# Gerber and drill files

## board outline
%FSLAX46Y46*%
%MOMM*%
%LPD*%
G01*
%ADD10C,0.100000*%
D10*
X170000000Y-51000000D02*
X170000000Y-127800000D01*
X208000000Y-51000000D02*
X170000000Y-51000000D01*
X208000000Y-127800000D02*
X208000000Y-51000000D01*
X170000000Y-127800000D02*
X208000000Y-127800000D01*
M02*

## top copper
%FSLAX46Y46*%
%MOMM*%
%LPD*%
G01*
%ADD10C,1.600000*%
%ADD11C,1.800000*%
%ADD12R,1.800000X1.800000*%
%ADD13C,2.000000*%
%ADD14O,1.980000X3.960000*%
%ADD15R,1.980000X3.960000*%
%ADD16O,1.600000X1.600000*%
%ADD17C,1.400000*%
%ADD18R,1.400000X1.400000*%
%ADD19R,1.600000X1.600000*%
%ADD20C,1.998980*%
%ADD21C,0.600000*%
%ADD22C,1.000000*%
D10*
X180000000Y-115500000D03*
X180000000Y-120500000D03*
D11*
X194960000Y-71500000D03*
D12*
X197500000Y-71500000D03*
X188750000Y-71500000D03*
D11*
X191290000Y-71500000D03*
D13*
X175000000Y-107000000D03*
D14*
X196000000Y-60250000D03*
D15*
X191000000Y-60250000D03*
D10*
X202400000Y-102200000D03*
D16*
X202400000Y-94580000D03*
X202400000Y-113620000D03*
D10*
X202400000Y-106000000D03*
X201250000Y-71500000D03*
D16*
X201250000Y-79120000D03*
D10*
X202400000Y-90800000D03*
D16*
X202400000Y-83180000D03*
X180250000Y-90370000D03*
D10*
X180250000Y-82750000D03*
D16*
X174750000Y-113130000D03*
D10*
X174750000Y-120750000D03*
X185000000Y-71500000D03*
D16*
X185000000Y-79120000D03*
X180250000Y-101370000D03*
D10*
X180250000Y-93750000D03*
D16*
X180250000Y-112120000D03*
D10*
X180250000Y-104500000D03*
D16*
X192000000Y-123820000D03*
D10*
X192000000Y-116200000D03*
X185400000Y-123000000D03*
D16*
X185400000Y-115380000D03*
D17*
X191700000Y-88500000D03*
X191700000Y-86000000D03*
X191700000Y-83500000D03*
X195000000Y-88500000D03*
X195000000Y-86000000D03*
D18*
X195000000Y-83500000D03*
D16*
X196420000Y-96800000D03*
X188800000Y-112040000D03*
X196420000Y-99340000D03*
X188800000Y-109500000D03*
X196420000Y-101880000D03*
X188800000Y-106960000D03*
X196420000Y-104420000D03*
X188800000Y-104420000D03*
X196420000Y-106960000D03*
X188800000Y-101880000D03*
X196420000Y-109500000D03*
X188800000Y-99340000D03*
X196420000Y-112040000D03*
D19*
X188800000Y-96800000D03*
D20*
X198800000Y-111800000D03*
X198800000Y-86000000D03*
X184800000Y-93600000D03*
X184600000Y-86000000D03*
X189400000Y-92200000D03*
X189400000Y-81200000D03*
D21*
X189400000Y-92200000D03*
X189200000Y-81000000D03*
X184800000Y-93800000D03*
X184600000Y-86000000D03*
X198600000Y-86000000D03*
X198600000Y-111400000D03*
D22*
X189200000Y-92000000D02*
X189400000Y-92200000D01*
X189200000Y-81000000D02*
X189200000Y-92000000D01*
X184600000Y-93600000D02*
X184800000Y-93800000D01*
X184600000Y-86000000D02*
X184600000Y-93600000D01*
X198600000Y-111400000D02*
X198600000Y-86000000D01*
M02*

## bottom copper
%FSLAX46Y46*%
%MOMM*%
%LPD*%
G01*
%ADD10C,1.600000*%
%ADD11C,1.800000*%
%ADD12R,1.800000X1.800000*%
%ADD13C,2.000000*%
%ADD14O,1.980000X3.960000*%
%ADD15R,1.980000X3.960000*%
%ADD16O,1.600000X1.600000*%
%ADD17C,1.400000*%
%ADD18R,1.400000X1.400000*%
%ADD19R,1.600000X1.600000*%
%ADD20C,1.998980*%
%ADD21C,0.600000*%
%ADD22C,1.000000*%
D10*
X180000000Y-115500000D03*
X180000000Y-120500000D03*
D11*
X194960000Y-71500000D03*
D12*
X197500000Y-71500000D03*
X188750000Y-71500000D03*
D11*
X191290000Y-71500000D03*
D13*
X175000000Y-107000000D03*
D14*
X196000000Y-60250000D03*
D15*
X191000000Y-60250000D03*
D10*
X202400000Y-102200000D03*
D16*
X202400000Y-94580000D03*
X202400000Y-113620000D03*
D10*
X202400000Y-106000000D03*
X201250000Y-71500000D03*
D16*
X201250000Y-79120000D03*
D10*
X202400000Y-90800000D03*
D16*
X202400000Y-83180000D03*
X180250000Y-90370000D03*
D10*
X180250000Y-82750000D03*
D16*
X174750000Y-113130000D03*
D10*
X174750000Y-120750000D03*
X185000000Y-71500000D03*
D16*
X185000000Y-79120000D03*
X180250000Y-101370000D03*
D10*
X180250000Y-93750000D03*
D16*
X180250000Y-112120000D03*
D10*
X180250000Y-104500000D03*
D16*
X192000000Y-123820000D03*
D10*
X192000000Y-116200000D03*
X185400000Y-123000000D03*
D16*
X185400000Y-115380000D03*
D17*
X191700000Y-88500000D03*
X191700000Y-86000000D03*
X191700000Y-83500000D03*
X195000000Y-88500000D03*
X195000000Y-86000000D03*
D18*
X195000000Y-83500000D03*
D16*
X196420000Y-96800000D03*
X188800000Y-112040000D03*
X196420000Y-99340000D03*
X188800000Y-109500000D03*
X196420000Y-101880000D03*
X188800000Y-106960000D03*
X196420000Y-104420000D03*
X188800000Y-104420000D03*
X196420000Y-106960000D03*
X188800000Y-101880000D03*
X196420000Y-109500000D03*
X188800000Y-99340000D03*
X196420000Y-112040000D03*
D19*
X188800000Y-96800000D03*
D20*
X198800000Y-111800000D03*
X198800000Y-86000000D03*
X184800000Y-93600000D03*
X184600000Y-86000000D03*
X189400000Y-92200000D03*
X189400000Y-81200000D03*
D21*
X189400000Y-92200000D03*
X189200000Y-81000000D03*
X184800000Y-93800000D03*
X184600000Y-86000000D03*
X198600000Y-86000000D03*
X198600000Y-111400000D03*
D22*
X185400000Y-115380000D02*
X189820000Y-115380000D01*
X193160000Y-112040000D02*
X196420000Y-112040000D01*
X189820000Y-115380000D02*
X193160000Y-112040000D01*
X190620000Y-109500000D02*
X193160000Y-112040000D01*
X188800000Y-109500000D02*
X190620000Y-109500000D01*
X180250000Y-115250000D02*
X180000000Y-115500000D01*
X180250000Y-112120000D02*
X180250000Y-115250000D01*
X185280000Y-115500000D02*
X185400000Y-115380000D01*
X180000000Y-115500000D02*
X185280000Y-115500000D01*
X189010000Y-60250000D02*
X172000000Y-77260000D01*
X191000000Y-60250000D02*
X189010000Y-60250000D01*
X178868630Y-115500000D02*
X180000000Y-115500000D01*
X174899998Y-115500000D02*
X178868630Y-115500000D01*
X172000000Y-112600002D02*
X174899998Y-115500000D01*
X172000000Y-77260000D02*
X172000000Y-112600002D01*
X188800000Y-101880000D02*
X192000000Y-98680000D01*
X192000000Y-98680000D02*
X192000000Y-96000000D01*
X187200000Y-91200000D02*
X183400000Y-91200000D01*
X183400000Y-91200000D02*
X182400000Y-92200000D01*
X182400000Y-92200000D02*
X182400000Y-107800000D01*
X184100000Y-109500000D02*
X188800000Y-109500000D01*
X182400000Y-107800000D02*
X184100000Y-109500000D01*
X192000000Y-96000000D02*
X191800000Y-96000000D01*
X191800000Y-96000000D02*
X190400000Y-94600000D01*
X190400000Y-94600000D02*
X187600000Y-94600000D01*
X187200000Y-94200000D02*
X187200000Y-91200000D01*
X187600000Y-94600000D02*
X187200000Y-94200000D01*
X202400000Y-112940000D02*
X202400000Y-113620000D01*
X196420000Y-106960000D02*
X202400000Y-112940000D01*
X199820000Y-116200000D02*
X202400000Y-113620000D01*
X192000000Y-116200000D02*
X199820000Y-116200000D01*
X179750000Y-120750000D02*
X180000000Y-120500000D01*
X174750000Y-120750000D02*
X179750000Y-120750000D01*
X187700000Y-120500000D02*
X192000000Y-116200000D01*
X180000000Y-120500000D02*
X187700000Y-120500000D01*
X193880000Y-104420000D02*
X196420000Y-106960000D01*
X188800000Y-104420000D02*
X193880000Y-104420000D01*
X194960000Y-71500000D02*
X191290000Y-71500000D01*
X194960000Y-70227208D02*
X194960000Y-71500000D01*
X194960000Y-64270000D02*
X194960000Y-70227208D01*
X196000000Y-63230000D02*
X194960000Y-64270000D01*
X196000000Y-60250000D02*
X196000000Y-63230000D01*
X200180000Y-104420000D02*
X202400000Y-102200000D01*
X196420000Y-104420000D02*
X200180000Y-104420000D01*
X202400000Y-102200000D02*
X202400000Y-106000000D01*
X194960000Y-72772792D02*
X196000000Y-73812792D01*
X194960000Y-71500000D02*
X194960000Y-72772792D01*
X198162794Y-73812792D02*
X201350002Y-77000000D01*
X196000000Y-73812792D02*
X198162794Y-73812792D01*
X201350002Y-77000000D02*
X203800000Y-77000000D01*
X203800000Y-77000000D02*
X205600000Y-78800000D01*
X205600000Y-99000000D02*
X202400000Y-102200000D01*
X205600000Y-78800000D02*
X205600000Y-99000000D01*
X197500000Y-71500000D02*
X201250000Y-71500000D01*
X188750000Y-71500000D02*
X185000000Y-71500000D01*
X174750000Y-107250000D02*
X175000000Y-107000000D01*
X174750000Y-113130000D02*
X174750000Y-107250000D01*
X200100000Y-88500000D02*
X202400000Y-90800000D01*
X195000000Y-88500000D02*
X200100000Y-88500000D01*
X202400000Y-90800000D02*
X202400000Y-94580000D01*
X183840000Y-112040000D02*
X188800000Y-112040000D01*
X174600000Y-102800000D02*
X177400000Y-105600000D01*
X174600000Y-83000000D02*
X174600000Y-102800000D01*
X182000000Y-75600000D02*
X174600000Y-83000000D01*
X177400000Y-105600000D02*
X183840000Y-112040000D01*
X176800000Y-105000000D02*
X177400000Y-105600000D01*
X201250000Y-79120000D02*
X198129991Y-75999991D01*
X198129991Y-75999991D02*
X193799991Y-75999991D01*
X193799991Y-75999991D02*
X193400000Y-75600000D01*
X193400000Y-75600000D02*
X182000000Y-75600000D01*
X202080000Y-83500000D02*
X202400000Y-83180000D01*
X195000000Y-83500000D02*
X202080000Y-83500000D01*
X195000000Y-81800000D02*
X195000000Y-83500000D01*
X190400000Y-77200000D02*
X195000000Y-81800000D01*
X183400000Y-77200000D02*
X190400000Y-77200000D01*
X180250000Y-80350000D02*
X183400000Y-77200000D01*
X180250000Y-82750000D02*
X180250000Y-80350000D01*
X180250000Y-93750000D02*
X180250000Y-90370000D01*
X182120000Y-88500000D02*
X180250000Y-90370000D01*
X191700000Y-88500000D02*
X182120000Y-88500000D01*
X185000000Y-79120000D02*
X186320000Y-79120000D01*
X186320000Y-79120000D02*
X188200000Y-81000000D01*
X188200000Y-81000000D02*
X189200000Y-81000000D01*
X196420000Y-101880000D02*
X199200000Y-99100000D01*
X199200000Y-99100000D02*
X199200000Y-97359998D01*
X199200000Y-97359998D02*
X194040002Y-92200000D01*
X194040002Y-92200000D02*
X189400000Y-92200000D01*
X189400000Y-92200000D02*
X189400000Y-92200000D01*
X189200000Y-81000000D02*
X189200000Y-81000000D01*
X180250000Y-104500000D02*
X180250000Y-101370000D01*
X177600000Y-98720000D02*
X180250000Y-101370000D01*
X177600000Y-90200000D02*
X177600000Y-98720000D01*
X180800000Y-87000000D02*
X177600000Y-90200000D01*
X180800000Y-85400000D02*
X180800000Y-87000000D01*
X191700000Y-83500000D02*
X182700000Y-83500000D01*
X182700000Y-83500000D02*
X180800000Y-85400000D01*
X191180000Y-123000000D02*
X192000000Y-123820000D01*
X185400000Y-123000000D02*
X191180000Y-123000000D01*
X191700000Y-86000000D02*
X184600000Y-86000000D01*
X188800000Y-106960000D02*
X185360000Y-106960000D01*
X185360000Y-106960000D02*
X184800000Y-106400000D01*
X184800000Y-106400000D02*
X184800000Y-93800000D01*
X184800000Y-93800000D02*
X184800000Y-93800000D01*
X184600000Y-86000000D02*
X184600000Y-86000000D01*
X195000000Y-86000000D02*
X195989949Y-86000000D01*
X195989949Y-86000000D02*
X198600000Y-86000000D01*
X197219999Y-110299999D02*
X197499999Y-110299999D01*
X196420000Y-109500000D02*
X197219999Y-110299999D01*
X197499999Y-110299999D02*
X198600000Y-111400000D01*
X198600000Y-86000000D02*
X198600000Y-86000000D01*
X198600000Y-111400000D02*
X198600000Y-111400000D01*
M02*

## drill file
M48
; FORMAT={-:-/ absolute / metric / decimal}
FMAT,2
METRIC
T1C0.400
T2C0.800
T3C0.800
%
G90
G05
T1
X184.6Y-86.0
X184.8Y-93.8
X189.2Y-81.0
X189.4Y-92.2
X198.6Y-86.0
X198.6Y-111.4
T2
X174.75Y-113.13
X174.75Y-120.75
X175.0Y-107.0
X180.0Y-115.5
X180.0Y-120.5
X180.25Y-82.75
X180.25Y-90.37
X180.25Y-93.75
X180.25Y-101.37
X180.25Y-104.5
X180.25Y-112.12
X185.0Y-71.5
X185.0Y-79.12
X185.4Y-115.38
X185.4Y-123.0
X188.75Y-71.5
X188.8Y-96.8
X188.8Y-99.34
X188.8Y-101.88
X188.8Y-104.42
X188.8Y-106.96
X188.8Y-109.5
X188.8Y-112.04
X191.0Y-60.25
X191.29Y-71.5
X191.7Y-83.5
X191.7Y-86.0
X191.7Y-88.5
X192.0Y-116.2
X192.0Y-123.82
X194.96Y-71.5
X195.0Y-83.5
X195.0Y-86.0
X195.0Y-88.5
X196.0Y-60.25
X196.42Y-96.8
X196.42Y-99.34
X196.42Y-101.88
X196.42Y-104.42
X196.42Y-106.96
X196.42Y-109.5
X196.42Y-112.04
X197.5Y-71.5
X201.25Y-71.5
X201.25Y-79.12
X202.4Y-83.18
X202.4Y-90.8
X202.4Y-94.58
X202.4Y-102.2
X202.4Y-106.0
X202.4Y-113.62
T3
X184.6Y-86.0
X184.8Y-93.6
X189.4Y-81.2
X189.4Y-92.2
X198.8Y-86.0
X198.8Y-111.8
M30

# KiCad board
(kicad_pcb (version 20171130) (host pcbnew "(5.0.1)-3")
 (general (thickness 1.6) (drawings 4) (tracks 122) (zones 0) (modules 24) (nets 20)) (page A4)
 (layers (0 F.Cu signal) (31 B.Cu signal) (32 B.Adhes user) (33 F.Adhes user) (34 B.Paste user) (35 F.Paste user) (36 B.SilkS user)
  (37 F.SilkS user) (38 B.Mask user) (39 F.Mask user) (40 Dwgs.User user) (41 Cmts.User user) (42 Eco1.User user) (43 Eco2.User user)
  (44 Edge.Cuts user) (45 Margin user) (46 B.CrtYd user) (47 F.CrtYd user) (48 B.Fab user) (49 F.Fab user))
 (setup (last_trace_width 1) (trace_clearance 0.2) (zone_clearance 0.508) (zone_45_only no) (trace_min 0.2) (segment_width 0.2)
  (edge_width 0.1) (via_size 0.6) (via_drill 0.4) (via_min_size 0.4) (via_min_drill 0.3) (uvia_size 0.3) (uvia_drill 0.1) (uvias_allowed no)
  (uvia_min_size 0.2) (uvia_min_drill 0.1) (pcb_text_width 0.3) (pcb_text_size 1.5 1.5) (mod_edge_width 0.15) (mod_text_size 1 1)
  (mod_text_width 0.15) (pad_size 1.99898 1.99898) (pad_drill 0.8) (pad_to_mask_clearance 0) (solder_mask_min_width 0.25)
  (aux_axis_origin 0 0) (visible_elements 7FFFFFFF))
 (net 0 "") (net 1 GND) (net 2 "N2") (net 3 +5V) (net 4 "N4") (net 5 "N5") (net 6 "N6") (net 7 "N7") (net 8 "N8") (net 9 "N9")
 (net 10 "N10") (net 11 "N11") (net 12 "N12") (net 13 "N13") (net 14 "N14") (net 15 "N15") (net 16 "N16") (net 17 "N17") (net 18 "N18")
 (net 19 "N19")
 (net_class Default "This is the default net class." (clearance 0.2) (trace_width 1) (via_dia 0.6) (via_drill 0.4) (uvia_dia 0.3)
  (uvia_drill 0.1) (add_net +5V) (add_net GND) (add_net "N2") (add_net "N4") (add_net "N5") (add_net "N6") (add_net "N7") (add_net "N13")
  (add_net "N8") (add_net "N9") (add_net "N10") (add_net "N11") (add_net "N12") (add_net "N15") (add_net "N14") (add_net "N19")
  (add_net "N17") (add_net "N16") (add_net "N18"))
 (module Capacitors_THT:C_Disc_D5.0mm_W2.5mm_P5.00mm (layer F.Cu) (at 180 120.5 90)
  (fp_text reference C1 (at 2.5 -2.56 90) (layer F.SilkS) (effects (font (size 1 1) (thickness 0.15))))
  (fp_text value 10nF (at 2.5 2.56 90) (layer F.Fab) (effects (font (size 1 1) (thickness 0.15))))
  (pad 2 thru_hole circle (at 5 0 90) (size 1.6 1.6) (drill 0.8) (layers *.Cu *.Mask) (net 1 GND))
  (pad 1 thru_hole circle (at 0 0 90) (size 1.6 1.6) (drill 0.8) (layers *.Cu *.Mask) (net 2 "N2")))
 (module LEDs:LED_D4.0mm (layer F.Cu) (at 197.5 71.5 180)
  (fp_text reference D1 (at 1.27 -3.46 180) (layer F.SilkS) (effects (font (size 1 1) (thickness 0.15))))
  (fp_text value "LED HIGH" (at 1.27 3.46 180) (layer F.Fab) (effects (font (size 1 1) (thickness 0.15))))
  (pad 2 thru_hole circle (at 2.54 0 180) (size 1.8 1.8) (drill 0.8) (layers *.Cu *.Mask) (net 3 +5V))
  (pad 1 thru_hole rect (at 0 0 180) (size 1.8 1.8) (drill 0.8) (layers *.Cu *.Mask) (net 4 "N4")))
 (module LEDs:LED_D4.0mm (layer F.Cu) (at 188.75 71.5)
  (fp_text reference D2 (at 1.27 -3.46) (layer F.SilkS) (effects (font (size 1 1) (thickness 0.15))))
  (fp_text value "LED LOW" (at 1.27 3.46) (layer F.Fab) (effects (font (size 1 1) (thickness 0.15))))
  (pad 1 thru_hole rect (at 0 0) (size 1.8 1.8) (drill 0.8) (layers *.Cu *.Mask) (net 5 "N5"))
  (pad 2 thru_hole circle (at 2.54 0) (size 1.8 1.8) (drill 0.8) (layers *.Cu *.Mask) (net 3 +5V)))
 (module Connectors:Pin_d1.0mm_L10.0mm (layer F.Cu) (at 175 107)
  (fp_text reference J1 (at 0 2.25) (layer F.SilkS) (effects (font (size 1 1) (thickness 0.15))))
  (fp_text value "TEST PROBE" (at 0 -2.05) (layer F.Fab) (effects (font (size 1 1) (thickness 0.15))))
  (pad 1 thru_hole circle (at 0 0) (size 2 2) (drill 0.8) (layers *.Cu *.Mask) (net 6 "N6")))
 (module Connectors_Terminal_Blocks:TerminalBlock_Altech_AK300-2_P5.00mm (layer F.Cu) (at 191 60.25)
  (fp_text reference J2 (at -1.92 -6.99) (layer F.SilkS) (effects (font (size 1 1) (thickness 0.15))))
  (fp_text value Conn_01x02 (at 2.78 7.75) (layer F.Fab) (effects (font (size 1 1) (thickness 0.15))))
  (pad 2 thru_hole oval (at 5 0) (size 1.98 3.96) (drill 0.8) (layers *.Cu *.Mask) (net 3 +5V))
  (pad 1 thru_hole rect (at 0 0) (size 1.98 3.96) (drill 0.8) (layers *.Cu *.Mask) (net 1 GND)))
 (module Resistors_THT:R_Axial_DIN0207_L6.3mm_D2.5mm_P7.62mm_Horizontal (layer F.Cu) (at 202.4 102.2 90)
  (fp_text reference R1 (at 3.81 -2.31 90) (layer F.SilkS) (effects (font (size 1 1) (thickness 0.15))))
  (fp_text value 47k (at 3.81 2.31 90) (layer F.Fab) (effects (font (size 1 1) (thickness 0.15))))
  (pad 1 thru_hole circle (at 0 0 90) (size 1.6 1.6) (drill 0.8) (layers *.Cu *.Mask) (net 3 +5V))
  (pad 2 thru_hole oval (at 7.62 0 90) (size 1.6 1.6) (drill 0.8) (layers *.Cu *.Mask) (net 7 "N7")))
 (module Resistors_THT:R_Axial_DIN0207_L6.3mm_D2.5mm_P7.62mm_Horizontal (layer F.Cu) (at 202.4 106 270)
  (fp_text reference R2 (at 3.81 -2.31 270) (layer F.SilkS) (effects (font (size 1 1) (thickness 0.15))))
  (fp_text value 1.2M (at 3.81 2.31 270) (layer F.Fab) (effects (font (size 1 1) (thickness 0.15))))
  (pad 2 thru_hole oval (at 7.62 0 270) (size 1.6 1.6) (drill 0.8) (layers *.Cu *.Mask) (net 2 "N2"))
  (pad 1 thru_hole circle (at 0 0 270) (size 1.6 1.6) (drill 0.8) (layers *.Cu *.Mask) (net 3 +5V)))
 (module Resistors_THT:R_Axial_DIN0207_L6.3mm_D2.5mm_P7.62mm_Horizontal (layer F.Cu) (at 201.25 71.5 270)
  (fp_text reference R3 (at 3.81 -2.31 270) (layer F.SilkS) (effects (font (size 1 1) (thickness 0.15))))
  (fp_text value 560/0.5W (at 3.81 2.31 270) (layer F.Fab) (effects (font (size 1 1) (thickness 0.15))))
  (pad 1 thru_hole circle (at 0 0 270) (size 1.6 1.6) (drill 0.8) (layers *.Cu *.Mask) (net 4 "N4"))
  (pad 2 thru_hole oval (at 7.62 0 270) (size 1.6 1.6) (drill 0.8) (layers *.Cu *.Mask) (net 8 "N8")))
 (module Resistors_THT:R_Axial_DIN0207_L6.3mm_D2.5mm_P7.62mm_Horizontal (layer F.Cu) (at 202.4 90.8 90)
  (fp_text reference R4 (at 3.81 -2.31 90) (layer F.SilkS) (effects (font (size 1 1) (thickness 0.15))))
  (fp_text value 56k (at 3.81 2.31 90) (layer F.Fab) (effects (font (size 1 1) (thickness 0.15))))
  (pad 1 thru_hole circle (at 0 0 90) (size 1.6 1.6) (drill 0.8) (layers *.Cu *.Mask) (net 7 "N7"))
  (pad 2 thru_hole oval (at 7.62 0 90) (size 1.6 1.6) (drill 0.8) (layers *.Cu *.Mask) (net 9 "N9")))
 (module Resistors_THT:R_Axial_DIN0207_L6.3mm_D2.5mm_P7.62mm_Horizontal (layer F.Cu) (at 180.25 82.75 270)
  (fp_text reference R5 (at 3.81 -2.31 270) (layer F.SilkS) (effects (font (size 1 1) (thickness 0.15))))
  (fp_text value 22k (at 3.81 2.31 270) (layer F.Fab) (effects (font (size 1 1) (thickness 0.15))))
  (pad 2 thru_hole oval (at 7.62 0 270) (size 1.6 1.6) (drill 0.8) (layers *.Cu *.Mask) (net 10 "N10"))
  (pad 1 thru_hole circle (at 0 0 270) (size 1.6 1.6) (drill 0.8) (layers *.Cu *.Mask) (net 9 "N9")))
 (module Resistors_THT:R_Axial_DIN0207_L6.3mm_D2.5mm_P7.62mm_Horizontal (layer F.Cu) (at 174.75 120.75 90)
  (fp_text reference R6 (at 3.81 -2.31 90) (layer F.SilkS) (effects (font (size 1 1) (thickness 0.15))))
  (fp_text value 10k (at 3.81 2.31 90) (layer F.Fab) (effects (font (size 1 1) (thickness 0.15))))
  (pad 2 thru_hole oval (at 7.62 0 90) (size 1.6 1.6) (drill 0.8) (layers *.Cu *.Mask) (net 6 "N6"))
  (pad 1 thru_hole circle (at 0 0 90) (size 1.6 1.6) (drill 0.8) (layers *.Cu *.Mask) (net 2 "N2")))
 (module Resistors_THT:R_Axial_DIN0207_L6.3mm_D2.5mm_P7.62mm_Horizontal (layer F.Cu) (at 185 71.5 270)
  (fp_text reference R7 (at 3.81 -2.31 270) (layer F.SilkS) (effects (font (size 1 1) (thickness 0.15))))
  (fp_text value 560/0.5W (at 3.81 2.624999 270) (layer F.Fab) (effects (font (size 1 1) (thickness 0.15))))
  (pad 1 thru_hole circle (at 0 0 270) (size 1.6 1.6) (drill 0.8) (layers *.Cu *.Mask) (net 5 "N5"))
  (pad 2 thru_hole oval (at 7.62 0 270) (size 1.6 1.6) (drill 0.8) (layers *.Cu *.Mask) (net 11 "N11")))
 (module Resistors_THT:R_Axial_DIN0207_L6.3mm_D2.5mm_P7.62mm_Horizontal (layer F.Cu) (at 180.25 93.75 270)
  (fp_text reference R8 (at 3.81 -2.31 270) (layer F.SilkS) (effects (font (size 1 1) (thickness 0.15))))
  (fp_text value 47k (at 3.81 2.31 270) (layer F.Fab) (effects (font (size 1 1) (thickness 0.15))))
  (pad 2 thru_hole oval (at 7.62 0 270) (size 1.6 1.6) (drill 0.8) (layers *.Cu *.Mask) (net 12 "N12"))
  (pad 1 thru_hole circle (at 0 0 270) (size 1.6 1.6) (drill 0.8) (layers *.Cu *.Mask) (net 10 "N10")))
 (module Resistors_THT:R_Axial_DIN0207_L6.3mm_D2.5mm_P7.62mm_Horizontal (layer F.Cu) (at 180.25 104.5 270)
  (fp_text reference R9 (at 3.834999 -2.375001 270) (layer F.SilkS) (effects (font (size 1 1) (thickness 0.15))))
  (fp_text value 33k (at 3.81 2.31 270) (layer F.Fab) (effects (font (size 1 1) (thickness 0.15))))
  (pad 2 thru_hole oval (at 7.62 0 270) (size 1.6 1.6) (drill 0.8) (layers *.Cu *.Mask) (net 1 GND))
  (pad 1 thru_hole circle (at 0 0 270) (size 1.6 1.6) (drill 0.8) (layers *.Cu *.Mask) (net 12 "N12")))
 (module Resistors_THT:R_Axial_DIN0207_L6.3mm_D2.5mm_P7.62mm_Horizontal (layer F.Cu) (at 192 116.2 270)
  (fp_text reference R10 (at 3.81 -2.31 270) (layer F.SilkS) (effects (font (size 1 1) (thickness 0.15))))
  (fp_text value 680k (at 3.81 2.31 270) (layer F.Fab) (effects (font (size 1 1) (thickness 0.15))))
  (pad 2 thru_hole oval (at 7.62 0 270) (size 1.6 1.6) (drill 0.8) (layers *.Cu *.Mask) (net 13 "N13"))
  (pad 1 thru_hole circle (at 0 0 270) (size 1.6 1.6) (drill 0.8) (layers *.Cu *.Mask) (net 2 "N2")))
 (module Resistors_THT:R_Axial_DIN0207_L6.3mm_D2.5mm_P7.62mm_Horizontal (layer F.Cu) (at 185.4 123 90)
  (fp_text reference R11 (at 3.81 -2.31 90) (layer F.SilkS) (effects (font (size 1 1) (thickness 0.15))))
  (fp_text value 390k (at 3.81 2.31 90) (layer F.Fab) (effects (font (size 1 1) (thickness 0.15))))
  (pad 1 thru_hole circle (at 0 0 90) (size 1.6 1.6) (drill 0.8) (layers *.Cu *.Mask) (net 13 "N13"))
  (pad 2 thru_hole oval (at 7.62 0 90) (size 1.6 1.6) (drill 0.8) (layers *.Cu *.Mask) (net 1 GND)))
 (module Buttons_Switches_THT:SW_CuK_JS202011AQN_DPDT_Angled (layer F.Cu) (at 195 83.5 270)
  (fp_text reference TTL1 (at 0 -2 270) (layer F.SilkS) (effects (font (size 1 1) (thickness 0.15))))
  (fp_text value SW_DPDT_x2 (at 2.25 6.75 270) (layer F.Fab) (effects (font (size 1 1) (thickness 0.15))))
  (pad 6 thru_hole circle (at 5 3.3 270) (size 1.4 1.4) (drill 0.8) (layers *.Cu *.Mask) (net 10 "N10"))
  (pad 5 thru_hole circle (at 2.5 3.3 270) (size 1.4 1.4) (drill 0.8) (layers *.Cu *.Mask) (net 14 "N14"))
  (pad 4 thru_hole circle (at 0 3.3 270) (size 1.4 1.4) (drill 0.8) (layers *.Cu *.Mask) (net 12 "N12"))
  (pad 3 thru_hole circle (at 5 0 270) (size 1.4 1.4) (drill 0.8) (layers *.Cu *.Mask) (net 7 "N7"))
  (pad 2 thru_hole circle (at 2.5 0 270) (size 1.4 1.4) (drill 0.8) (layers *.Cu *.Mask) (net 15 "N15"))
  (pad 1 thru_hole rect (at 0 0 270) (size 1.4 1.4) (drill 0.8) (layers *.Cu *.Mask) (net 9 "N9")))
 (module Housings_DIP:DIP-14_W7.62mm (layer F.Cu) (at 188.8 96.8)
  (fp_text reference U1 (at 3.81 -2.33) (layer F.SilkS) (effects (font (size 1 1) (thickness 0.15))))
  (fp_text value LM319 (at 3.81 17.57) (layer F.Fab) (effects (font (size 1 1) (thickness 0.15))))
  (pad 14 thru_hole oval (at 7.62 0) (size 1.6 1.6) (drill 0.8) (layers *.Cu *.Mask) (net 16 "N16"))
  (pad 7 thru_hole oval (at 0 15.24) (size 1.6 1.6) (drill 0.8) (layers *.Cu *.Mask) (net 8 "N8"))
  (pad 13 thru_hole oval (at 7.62 2.54) (size 1.6 1.6) (drill 0.8) (layers *.Cu *.Mask) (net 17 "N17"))
  (pad 6 thru_hole oval (at 0 12.7) (size 1.6 1.6) (drill 0.8) (layers *.Cu *.Mask) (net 1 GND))
  (pad 12 thru_hole oval (at 7.62 5.08) (size 1.6 1.6) (drill 0.8) (layers *.Cu *.Mask) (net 11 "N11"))
  (pad 5 thru_hole oval (at 0 10.16) (size 1.6 1.6) (drill 0.8) (layers *.Cu *.Mask) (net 14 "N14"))
  (pad 11 thru_hole oval (at 7.62 7.62) (size 1.6 1.6) (drill 0.8) (layers *.Cu *.Mask) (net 3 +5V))
  (pad 4 thru_hole oval (at 0 7.62) (size 1.6 1.6) (drill 0.8) (layers *.Cu *.Mask) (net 2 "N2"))
  (pad 10 thru_hole oval (at 7.62 10.16) (size 1.6 1.6) (drill 0.8) (layers *.Cu *.Mask) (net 2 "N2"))
  (pad 3 thru_hole oval (at 0 5.08) (size 1.6 1.6) (drill 0.8) (layers *.Cu *.Mask) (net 1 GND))
  (pad 9 thru_hole oval (at 7.62 12.7) (size 1.6 1.6) (drill 0.8) (layers *.Cu *.Mask) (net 15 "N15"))
  (pad 2 thru_hole oval (at 0 2.54) (size 1.6 1.6) (drill 0.8) (layers *.Cu *.Mask) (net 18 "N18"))
  (pad 8 thru_hole oval (at 7.62 15.24) (size 1.6 1.6) (drill 0.8) (layers *.Cu *.Mask) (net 1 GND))
  (pad 1 thru_hole rect (at 0 0) (size 1.6 1.6) (drill 0.8) (layers *.Cu *.Mask) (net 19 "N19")))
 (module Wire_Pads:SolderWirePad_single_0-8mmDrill (layer F.Cu) (at 198.8 111.8)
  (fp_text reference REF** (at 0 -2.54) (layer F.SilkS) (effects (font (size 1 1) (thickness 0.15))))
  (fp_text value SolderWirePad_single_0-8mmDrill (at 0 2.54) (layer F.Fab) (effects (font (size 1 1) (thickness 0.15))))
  (pad 1 thru_hole circle (at 0 0) (size 1.99898 1.99898) (drill 0.8001) (layers *.Cu *.Mask)))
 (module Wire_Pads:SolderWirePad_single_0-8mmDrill (layer F.Cu) (at 198.8 86)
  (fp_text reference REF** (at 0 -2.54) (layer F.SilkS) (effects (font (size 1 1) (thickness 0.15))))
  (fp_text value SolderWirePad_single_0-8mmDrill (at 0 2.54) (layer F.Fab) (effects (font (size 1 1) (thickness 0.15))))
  (pad 1 thru_hole circle (at 0 0) (size 1.99898 1.99898) (drill 0.8001) (layers *.Cu *.Mask)))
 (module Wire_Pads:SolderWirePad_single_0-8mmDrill (layer F.Cu) (at 184.8 93.6)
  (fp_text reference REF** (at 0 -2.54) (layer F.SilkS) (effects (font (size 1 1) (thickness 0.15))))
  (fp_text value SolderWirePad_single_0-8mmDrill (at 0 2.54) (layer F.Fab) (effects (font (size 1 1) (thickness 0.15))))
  (pad 1 thru_hole circle (at 0 0) (size 1.99898 1.99898) (drill 0.8001) (layers *.Cu *.Mask)))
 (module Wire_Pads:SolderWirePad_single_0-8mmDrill (layer F.Cu) (at 184.6 86)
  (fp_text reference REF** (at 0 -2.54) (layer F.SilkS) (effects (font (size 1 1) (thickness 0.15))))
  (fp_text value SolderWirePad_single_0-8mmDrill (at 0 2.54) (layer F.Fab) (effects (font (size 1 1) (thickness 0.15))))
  (pad 1 thru_hole circle (at 0 0) (size 1.99898 1.99898) (drill 0.8001) (layers *.Cu *.Mask)))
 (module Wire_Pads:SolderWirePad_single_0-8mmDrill (layer F.Cu) (at 189.4 92.2)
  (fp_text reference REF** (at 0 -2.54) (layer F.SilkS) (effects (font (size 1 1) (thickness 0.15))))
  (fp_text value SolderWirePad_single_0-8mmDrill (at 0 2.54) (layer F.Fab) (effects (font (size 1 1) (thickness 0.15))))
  (pad 1 thru_hole circle (at 0 0) (size 1.99898 1.99898) (drill 0.8001) (layers *.Cu *.Mask)))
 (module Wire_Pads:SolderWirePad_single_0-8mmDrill (layer F.Cu) (at 189.4 81.2)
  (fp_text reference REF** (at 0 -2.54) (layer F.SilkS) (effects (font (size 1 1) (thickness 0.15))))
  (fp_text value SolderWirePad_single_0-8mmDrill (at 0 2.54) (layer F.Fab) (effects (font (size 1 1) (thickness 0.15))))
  (pad 1 thru_hole circle (at 0 0) (size 1.99898 1.99898) (drill 0.8001) (layers *.Cu *.Mask)))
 (gr_line (start 170 51) (end 170 127.8) (layer Edge.Cuts) (width 0.1))
 (gr_line (start 208 51) (end 170 51) (layer Edge.Cuts) (width 0.1))
 (gr_line (start 208 127.8) (end 208 51) (layer Edge.Cuts) (width 0.1))
 (gr_line (start 170 127.8) (end 208 127.8) (layer Edge.Cuts) (width 0.1))
 (segment (start 185.4 115.38) (end 189.82 115.38) (width 1) (layer B.Cu) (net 1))
 (segment (start 193.16 112.04) (end 196.42 112.04) (width 1) (layer B.Cu) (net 1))
 (segment (start 189.82 115.38) (end 193.16 112.04) (width 1) (layer B.Cu) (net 1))
 (segment (start 190.62 109.5) (end 193.16 112.04) (width 1) (layer B.Cu) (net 1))
 (segment (start 188.8 109.5) (end 190.62 109.5) (width 1) (layer B.Cu) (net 1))
 (segment (start 180.25 115.25) (end 180 115.5) (width 1) (layer B.Cu) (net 1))
 (segment (start 180.25 112.12) (end 180.25 115.25) (width 1) (layer B.Cu) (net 1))
 (segment (start 185.28 115.5) (end 185.4 115.38) (width 1) (layer B.Cu) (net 1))
 (segment (start 180 115.5) (end 185.28 115.5) (width 1) (layer B.Cu) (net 1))
 (segment (start 189.01 60.25) (end 172 77.26) (width 1) (layer B.Cu) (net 1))
 (segment (start 191 60.25) (end 189.01 60.25) (width 1) (layer B.Cu) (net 1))
 (segment (start 178.86863 115.5) (end 180 115.5) (width 1) (layer B.Cu) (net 1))
 (segment (start 174.899998 115.5) (end 178.86863 115.5) (width 1) (layer B.Cu) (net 1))
 (segment (start 172 112.600002) (end 174.899998 115.5) (width 1) (layer B.Cu) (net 1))
 (segment (start 172 77.26) (end 172 112.600002) (width 1) (layer B.Cu) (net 1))
 (segment (start 188.8 101.88) (end 192 98.68) (width 1) (layer B.Cu) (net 1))
 (segment (start 192 98.68) (end 192 96) (width 1) (layer B.Cu) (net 1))
 (segment (start 187.2 91.2) (end 183.4 91.2) (width 1) (layer B.Cu) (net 1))
 (segment (start 183.4 91.2) (end 182.4 92.2) (width 1) (layer B.Cu) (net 1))
 (segment (start 182.4 92.2) (end 182.4 107.8) (width 1) (layer B.Cu) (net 1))
 (segment (start 184.1 109.5) (end 188.8 109.5) (width 1) (layer B.Cu) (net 1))
 (segment (start 182.4 107.8) (end 184.1 109.5) (width 1) (layer B.Cu) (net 1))
 (segment (start 192 96) (end 191.8 96) (width 1) (layer B.Cu) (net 1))
 (segment (start 191.8 96) (end 190.4 94.6) (width 1) (layer B.Cu) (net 1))
 (segment (start 190.4 94.6) (end 187.6 94.6) (width 1) (layer B.Cu) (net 1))
 (segment (start 187.2 94.2) (end 187.2 91.2) (width 1) (layer B.Cu) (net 1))
 (segment (start 187.6 94.6) (end 187.2 94.2) (width 1) (layer B.Cu) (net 1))
 (segment (start 202.4 112.94) (end 202.4 113.62) (width 1) (layer B.Cu) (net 2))
 (segment (start 196.42 106.96) (end 202.4 112.94) (width 1) (layer B.Cu) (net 2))
 (segment (start 199.82 116.2) (end 202.4 113.62) (width 1) (layer B.Cu) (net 2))
 (segment (start 192 116.2) (end 199.82 116.2) (width 1) (layer B.Cu) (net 2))
 (segment (start 179.75 120.75) (end 180 120.5) (width 1) (layer B.Cu) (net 2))
 (segment (start 174.75 120.75) (end 179.75 120.75) (width 1) (layer B.Cu) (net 2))
 (segment (start 187.7 120.5) (end 192 116.2) (width 1) (layer B.Cu) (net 2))
 (segment (start 180 120.5) (end 187.7 120.5) (width 1) (layer B.Cu) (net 2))
 (segment (start 193.88 104.42) (end 196.42 106.96) (width 1) (layer B.Cu) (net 2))
 (segment (start 188.8 104.42) (end 193.88 104.42) (width 1) (layer B.Cu) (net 2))
 (segment (start 194.96 71.5) (end 191.29 71.5) (width 1) (layer B.Cu) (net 3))
 (segment (start 194.96 70.227208) (end 194.96 71.5) (width 1) (layer B.Cu) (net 3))
 (segment (start 194.96 64.27) (end 194.96 70.227208) (width 1) (layer B.Cu) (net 3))
 (segment (start 196 63.23) (end 194.96 64.27) (width 1) (layer B.Cu) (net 3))
 (segment (start 196 60.25) (end 196 63.23) (width 1) (layer B.Cu) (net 3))
 (segment (start 200.18 104.42) (end 202.4 102.2) (width 1) (layer B.Cu) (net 3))
 (segment (start 196.42 104.42) (end 200.18 104.42) (width 1) (layer B.Cu) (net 3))
 (segment (start 202.4 102.2) (end 202.4 106) (width 1) (layer B.Cu) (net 3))
 (segment (start 194.96 72.772792) (end 196 73.812792) (width 1) (layer B.Cu) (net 3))
 (segment (start 194.96 71.5) (end 194.96 72.772792) (width 1) (layer B.Cu) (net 3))
 (segment (start 198.162794 73.812792) (end 201.350002 77) (width 1) (layer B.Cu) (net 3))
 (segment (start 196 73.812792) (end 198.162794 73.812792) (width 1) (layer B.Cu) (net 3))
 (segment (start 201.350002 77) (end 203.8 77) (width 1) (layer B.Cu) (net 3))
 (segment (start 203.8 77) (end 205.6 78.8) (width 1) (layer B.Cu) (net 3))
 (segment (start 205.6 99) (end 202.4 102.2) (width 1) (layer B.Cu) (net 3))
 (segment (start 205.6 78.8) (end 205.6 99) (width 1) (layer B.Cu) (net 3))
 (segment (start 197.5 71.5) (end 201.25 71.5) (width 1) (layer B.Cu) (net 4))
 (segment (start 188.75 71.5) (end 185 71.5) (width 1) (layer B.Cu) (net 5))
 (segment (start 174.75 107.25) (end 175 107) (width 1) (layer B.Cu) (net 6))
 (segment (start 174.75 113.13) (end 174.75 107.25) (width 1) (layer B.Cu) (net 6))
 (segment (start 200.1 88.5) (end 202.4 90.8) (width 1) (layer B.Cu) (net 7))
 (segment (start 195 88.5) (end 200.1 88.5) (width 1) (layer B.Cu) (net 7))
 (segment (start 202.4 90.8) (end 202.4 94.58) (width 1) (layer B.Cu) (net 7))
 (segment (start 183.84 112.04) (end 188.8 112.04) (width 1) (layer B.Cu) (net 8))
 (segment (start 174.6 102.8) (end 177.4 105.6) (width 1) (layer B.Cu) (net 8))
 (segment (start 174.6 83) (end 174.6 102.8) (width 1) (layer B.Cu) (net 8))
 (segment (start 182 75.6) (end 174.6 83) (width 1) (layer B.Cu) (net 8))
 (segment (start 177.4 105.6) (end 183.84 112.04) (width 1) (layer B.Cu) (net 8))
 (segment (start 176.8 105) (end 177.4 105.6) (width 1) (layer B.Cu) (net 8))
 (segment (start 201.25 79.12) (end 198.129991 75.999991) (width 1) (layer B.Cu) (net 8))
 (segment (start 198.129991 75.999991) (end 193.799991 75.999991) (width 1) (layer B.Cu) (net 8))
 (segment (start 193.799991 75.999991) (end 193.4 75.6) (width 1) (layer B.Cu) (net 8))
 (segment (start 193.4 75.6) (end 182 75.6) (width 1) (layer B.Cu) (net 8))
 (segment (start 202.08 83.5) (end 202.4 83.18) (width 1) (layer B.Cu) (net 9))
 (segment (start 195 83.5) (end 202.08 83.5) (width 1) (layer B.Cu) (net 9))
 (segment (start 195 81.8) (end 195 83.5) (width 1) (layer B.Cu) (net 9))
 (segment (start 190.4 77.2) (end 195 81.8) (width 1) (layer B.Cu) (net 9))
 (segment (start 183.4 77.2) (end 190.4 77.2) (width 1) (layer B.Cu) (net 9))
 (segment (start 180.25 80.35) (end 183.4 77.2) (width 1) (layer B.Cu) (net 9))
 (segment (start 180.25 82.75) (end 180.25 80.35) (width 1) (layer B.Cu) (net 9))
 (segment (start 180.25 93.75) (end 180.25 90.37) (width 1) (layer B.Cu) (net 10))
 (segment (start 182.12 88.5) (end 180.25 90.37) (width 1) (layer B.Cu) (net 10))
 (segment (start 191.7 88.5) (end 182.12 88.5) (width 1) (layer B.Cu) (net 10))
 (segment (start 185 79.12) (end 186.32 79.12) (width 1) (layer B.Cu) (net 11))
 (segment (start 186.32 79.12) (end 188.2 81) (width 1) (layer B.Cu) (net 11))
 (segment (start 188.2 81) (end 189.2 81) (width 1) (layer B.Cu) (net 11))
 (segment (start 196.42 101.88) (end 199.2 99.1) (width 1) (layer B.Cu) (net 11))
 (segment (start 199.2 99.1) (end 199.2 97.359998) (width 1) (layer B.Cu) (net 11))
 (segment (start 199.2 97.359998) (end 194.040002 92.2) (width 1) (layer B.Cu) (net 11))
 (segment (start 194.040002 92.2) (end 189.4 92.2) (width 1) (layer B.Cu) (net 11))
 (segment (start 189.4 92.2) (end 189.4 92.2) (width 1) (layer B.Cu) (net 11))
 (via (at 189.4 92.2) (size 0.6) (drill 0.4) (layers F.Cu B.Cu) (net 11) (status 1000000))
 (segment (start 189.2 81) (end 189.2 81) (width 1) (layer B.Cu) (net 11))
 (via (at 189.2 81) (size 0.6) (drill 0.4) (layers F.Cu B.Cu) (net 11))
 (segment (start 189.2 92) (end 189.4 92.2) (width 1) (layer F.Cu) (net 11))
 (segment (start 189.2 81) (end 189.2 92) (width 1) (layer F.Cu) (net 11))
 (segment (start 180.25 104.5) (end 180.25 101.37) (width 1) (layer B.Cu) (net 12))
 (segment (start 177.6 98.72) (end 180.25 101.37) (width 1) (layer B.Cu) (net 12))
 (segment (start 177.6 90.2) (end 177.6 98.72) (width 1) (layer B.Cu) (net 12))
 (segment (start 180.8 87) (end 177.6 90.2) (width 1) (layer B.Cu) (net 12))
 (segment (start 180.8 85.4) (end 180.8 87) (width 1) (layer B.Cu) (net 12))
 (segment (start 191.7 83.5) (end 182.7 83.5) (width 1) (layer B.Cu) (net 12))
 (segment (start 182.7 83.5) (end 180.8 85.4) (width 1) (layer B.Cu) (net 12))
 (segment (start 191.18 123) (end 192 123.82) (width 1) (layer B.Cu) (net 13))
 (segment (start 185.4 123) (end 191.18 123) (width 1) (layer B.Cu) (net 13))
 (segment (start 191.7 86) (end 184.6 86) (width 1) (layer B.Cu) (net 14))
 (segment (start 188.8 106.96) (end 185.36 106.96) (width 1) (layer B.Cu) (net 14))
 (segment (start 185.36 106.96) (end 184.8 106.4) (width 1) (layer B.Cu) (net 14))
 (segment (start 184.8 106.4) (end 184.8 93.8) (width 1) (layer B.Cu) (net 14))
 (segment (start 184.8 93.8) (end 184.8 93.8) (width 1) (layer B.Cu) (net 14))
 (via (at 184.8 93.8) (size 0.6) (drill 0.4) (layers F.Cu B.Cu) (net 14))
 (segment (start 184.6 86) (end 184.6 86) (width 1) (layer B.Cu) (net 14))
 (via (at 184.6 86) (size 0.6) (drill 0.4) (layers F.Cu B.Cu) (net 14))
 (segment (start 184.6 93.6) (end 184.8 93.8) (width 1) (layer F.Cu) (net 14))
 (segment (start 184.6 86) (end 184.6 93.6) (width 1) (layer F.Cu) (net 14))
 (segment (start 195 86) (end 195.989949 86) (width 1) (layer B.Cu) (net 15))
 (segment (start 195.989949 86) (end 198.6 86) (width 1) (layer B.Cu) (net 15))
 (segment (start 197.219999 110.299999) (end 197.499999 110.299999) (width 1) (layer B.Cu) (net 15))
 (segment (start 196.42 109.5) (end 197.219999 110.299999) (width 1) (layer B.Cu) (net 15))
 (segment (start 197.499999 110.299999) (end 198.6 111.4) (width 1) (layer B.Cu) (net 15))
 (segment (start 198.6 86) (end 198.6 86) (width 1) (layer B.Cu) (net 15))
 (via (at 198.6 86) (size 0.6) (drill 0.4) (layers F.Cu B.Cu) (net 15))
 (segment (start 198.6 111.4) (end 198.6 111.4) (width 1) (layer B.Cu) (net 15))
 (via (at 198.6 111.4) (size 0.6) (drill 0.4) (layers F.Cu B.Cu) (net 15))
 (segment (start 198.6 111.4) (end 198.6 86) (width 1) (layer F.Cu) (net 15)))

